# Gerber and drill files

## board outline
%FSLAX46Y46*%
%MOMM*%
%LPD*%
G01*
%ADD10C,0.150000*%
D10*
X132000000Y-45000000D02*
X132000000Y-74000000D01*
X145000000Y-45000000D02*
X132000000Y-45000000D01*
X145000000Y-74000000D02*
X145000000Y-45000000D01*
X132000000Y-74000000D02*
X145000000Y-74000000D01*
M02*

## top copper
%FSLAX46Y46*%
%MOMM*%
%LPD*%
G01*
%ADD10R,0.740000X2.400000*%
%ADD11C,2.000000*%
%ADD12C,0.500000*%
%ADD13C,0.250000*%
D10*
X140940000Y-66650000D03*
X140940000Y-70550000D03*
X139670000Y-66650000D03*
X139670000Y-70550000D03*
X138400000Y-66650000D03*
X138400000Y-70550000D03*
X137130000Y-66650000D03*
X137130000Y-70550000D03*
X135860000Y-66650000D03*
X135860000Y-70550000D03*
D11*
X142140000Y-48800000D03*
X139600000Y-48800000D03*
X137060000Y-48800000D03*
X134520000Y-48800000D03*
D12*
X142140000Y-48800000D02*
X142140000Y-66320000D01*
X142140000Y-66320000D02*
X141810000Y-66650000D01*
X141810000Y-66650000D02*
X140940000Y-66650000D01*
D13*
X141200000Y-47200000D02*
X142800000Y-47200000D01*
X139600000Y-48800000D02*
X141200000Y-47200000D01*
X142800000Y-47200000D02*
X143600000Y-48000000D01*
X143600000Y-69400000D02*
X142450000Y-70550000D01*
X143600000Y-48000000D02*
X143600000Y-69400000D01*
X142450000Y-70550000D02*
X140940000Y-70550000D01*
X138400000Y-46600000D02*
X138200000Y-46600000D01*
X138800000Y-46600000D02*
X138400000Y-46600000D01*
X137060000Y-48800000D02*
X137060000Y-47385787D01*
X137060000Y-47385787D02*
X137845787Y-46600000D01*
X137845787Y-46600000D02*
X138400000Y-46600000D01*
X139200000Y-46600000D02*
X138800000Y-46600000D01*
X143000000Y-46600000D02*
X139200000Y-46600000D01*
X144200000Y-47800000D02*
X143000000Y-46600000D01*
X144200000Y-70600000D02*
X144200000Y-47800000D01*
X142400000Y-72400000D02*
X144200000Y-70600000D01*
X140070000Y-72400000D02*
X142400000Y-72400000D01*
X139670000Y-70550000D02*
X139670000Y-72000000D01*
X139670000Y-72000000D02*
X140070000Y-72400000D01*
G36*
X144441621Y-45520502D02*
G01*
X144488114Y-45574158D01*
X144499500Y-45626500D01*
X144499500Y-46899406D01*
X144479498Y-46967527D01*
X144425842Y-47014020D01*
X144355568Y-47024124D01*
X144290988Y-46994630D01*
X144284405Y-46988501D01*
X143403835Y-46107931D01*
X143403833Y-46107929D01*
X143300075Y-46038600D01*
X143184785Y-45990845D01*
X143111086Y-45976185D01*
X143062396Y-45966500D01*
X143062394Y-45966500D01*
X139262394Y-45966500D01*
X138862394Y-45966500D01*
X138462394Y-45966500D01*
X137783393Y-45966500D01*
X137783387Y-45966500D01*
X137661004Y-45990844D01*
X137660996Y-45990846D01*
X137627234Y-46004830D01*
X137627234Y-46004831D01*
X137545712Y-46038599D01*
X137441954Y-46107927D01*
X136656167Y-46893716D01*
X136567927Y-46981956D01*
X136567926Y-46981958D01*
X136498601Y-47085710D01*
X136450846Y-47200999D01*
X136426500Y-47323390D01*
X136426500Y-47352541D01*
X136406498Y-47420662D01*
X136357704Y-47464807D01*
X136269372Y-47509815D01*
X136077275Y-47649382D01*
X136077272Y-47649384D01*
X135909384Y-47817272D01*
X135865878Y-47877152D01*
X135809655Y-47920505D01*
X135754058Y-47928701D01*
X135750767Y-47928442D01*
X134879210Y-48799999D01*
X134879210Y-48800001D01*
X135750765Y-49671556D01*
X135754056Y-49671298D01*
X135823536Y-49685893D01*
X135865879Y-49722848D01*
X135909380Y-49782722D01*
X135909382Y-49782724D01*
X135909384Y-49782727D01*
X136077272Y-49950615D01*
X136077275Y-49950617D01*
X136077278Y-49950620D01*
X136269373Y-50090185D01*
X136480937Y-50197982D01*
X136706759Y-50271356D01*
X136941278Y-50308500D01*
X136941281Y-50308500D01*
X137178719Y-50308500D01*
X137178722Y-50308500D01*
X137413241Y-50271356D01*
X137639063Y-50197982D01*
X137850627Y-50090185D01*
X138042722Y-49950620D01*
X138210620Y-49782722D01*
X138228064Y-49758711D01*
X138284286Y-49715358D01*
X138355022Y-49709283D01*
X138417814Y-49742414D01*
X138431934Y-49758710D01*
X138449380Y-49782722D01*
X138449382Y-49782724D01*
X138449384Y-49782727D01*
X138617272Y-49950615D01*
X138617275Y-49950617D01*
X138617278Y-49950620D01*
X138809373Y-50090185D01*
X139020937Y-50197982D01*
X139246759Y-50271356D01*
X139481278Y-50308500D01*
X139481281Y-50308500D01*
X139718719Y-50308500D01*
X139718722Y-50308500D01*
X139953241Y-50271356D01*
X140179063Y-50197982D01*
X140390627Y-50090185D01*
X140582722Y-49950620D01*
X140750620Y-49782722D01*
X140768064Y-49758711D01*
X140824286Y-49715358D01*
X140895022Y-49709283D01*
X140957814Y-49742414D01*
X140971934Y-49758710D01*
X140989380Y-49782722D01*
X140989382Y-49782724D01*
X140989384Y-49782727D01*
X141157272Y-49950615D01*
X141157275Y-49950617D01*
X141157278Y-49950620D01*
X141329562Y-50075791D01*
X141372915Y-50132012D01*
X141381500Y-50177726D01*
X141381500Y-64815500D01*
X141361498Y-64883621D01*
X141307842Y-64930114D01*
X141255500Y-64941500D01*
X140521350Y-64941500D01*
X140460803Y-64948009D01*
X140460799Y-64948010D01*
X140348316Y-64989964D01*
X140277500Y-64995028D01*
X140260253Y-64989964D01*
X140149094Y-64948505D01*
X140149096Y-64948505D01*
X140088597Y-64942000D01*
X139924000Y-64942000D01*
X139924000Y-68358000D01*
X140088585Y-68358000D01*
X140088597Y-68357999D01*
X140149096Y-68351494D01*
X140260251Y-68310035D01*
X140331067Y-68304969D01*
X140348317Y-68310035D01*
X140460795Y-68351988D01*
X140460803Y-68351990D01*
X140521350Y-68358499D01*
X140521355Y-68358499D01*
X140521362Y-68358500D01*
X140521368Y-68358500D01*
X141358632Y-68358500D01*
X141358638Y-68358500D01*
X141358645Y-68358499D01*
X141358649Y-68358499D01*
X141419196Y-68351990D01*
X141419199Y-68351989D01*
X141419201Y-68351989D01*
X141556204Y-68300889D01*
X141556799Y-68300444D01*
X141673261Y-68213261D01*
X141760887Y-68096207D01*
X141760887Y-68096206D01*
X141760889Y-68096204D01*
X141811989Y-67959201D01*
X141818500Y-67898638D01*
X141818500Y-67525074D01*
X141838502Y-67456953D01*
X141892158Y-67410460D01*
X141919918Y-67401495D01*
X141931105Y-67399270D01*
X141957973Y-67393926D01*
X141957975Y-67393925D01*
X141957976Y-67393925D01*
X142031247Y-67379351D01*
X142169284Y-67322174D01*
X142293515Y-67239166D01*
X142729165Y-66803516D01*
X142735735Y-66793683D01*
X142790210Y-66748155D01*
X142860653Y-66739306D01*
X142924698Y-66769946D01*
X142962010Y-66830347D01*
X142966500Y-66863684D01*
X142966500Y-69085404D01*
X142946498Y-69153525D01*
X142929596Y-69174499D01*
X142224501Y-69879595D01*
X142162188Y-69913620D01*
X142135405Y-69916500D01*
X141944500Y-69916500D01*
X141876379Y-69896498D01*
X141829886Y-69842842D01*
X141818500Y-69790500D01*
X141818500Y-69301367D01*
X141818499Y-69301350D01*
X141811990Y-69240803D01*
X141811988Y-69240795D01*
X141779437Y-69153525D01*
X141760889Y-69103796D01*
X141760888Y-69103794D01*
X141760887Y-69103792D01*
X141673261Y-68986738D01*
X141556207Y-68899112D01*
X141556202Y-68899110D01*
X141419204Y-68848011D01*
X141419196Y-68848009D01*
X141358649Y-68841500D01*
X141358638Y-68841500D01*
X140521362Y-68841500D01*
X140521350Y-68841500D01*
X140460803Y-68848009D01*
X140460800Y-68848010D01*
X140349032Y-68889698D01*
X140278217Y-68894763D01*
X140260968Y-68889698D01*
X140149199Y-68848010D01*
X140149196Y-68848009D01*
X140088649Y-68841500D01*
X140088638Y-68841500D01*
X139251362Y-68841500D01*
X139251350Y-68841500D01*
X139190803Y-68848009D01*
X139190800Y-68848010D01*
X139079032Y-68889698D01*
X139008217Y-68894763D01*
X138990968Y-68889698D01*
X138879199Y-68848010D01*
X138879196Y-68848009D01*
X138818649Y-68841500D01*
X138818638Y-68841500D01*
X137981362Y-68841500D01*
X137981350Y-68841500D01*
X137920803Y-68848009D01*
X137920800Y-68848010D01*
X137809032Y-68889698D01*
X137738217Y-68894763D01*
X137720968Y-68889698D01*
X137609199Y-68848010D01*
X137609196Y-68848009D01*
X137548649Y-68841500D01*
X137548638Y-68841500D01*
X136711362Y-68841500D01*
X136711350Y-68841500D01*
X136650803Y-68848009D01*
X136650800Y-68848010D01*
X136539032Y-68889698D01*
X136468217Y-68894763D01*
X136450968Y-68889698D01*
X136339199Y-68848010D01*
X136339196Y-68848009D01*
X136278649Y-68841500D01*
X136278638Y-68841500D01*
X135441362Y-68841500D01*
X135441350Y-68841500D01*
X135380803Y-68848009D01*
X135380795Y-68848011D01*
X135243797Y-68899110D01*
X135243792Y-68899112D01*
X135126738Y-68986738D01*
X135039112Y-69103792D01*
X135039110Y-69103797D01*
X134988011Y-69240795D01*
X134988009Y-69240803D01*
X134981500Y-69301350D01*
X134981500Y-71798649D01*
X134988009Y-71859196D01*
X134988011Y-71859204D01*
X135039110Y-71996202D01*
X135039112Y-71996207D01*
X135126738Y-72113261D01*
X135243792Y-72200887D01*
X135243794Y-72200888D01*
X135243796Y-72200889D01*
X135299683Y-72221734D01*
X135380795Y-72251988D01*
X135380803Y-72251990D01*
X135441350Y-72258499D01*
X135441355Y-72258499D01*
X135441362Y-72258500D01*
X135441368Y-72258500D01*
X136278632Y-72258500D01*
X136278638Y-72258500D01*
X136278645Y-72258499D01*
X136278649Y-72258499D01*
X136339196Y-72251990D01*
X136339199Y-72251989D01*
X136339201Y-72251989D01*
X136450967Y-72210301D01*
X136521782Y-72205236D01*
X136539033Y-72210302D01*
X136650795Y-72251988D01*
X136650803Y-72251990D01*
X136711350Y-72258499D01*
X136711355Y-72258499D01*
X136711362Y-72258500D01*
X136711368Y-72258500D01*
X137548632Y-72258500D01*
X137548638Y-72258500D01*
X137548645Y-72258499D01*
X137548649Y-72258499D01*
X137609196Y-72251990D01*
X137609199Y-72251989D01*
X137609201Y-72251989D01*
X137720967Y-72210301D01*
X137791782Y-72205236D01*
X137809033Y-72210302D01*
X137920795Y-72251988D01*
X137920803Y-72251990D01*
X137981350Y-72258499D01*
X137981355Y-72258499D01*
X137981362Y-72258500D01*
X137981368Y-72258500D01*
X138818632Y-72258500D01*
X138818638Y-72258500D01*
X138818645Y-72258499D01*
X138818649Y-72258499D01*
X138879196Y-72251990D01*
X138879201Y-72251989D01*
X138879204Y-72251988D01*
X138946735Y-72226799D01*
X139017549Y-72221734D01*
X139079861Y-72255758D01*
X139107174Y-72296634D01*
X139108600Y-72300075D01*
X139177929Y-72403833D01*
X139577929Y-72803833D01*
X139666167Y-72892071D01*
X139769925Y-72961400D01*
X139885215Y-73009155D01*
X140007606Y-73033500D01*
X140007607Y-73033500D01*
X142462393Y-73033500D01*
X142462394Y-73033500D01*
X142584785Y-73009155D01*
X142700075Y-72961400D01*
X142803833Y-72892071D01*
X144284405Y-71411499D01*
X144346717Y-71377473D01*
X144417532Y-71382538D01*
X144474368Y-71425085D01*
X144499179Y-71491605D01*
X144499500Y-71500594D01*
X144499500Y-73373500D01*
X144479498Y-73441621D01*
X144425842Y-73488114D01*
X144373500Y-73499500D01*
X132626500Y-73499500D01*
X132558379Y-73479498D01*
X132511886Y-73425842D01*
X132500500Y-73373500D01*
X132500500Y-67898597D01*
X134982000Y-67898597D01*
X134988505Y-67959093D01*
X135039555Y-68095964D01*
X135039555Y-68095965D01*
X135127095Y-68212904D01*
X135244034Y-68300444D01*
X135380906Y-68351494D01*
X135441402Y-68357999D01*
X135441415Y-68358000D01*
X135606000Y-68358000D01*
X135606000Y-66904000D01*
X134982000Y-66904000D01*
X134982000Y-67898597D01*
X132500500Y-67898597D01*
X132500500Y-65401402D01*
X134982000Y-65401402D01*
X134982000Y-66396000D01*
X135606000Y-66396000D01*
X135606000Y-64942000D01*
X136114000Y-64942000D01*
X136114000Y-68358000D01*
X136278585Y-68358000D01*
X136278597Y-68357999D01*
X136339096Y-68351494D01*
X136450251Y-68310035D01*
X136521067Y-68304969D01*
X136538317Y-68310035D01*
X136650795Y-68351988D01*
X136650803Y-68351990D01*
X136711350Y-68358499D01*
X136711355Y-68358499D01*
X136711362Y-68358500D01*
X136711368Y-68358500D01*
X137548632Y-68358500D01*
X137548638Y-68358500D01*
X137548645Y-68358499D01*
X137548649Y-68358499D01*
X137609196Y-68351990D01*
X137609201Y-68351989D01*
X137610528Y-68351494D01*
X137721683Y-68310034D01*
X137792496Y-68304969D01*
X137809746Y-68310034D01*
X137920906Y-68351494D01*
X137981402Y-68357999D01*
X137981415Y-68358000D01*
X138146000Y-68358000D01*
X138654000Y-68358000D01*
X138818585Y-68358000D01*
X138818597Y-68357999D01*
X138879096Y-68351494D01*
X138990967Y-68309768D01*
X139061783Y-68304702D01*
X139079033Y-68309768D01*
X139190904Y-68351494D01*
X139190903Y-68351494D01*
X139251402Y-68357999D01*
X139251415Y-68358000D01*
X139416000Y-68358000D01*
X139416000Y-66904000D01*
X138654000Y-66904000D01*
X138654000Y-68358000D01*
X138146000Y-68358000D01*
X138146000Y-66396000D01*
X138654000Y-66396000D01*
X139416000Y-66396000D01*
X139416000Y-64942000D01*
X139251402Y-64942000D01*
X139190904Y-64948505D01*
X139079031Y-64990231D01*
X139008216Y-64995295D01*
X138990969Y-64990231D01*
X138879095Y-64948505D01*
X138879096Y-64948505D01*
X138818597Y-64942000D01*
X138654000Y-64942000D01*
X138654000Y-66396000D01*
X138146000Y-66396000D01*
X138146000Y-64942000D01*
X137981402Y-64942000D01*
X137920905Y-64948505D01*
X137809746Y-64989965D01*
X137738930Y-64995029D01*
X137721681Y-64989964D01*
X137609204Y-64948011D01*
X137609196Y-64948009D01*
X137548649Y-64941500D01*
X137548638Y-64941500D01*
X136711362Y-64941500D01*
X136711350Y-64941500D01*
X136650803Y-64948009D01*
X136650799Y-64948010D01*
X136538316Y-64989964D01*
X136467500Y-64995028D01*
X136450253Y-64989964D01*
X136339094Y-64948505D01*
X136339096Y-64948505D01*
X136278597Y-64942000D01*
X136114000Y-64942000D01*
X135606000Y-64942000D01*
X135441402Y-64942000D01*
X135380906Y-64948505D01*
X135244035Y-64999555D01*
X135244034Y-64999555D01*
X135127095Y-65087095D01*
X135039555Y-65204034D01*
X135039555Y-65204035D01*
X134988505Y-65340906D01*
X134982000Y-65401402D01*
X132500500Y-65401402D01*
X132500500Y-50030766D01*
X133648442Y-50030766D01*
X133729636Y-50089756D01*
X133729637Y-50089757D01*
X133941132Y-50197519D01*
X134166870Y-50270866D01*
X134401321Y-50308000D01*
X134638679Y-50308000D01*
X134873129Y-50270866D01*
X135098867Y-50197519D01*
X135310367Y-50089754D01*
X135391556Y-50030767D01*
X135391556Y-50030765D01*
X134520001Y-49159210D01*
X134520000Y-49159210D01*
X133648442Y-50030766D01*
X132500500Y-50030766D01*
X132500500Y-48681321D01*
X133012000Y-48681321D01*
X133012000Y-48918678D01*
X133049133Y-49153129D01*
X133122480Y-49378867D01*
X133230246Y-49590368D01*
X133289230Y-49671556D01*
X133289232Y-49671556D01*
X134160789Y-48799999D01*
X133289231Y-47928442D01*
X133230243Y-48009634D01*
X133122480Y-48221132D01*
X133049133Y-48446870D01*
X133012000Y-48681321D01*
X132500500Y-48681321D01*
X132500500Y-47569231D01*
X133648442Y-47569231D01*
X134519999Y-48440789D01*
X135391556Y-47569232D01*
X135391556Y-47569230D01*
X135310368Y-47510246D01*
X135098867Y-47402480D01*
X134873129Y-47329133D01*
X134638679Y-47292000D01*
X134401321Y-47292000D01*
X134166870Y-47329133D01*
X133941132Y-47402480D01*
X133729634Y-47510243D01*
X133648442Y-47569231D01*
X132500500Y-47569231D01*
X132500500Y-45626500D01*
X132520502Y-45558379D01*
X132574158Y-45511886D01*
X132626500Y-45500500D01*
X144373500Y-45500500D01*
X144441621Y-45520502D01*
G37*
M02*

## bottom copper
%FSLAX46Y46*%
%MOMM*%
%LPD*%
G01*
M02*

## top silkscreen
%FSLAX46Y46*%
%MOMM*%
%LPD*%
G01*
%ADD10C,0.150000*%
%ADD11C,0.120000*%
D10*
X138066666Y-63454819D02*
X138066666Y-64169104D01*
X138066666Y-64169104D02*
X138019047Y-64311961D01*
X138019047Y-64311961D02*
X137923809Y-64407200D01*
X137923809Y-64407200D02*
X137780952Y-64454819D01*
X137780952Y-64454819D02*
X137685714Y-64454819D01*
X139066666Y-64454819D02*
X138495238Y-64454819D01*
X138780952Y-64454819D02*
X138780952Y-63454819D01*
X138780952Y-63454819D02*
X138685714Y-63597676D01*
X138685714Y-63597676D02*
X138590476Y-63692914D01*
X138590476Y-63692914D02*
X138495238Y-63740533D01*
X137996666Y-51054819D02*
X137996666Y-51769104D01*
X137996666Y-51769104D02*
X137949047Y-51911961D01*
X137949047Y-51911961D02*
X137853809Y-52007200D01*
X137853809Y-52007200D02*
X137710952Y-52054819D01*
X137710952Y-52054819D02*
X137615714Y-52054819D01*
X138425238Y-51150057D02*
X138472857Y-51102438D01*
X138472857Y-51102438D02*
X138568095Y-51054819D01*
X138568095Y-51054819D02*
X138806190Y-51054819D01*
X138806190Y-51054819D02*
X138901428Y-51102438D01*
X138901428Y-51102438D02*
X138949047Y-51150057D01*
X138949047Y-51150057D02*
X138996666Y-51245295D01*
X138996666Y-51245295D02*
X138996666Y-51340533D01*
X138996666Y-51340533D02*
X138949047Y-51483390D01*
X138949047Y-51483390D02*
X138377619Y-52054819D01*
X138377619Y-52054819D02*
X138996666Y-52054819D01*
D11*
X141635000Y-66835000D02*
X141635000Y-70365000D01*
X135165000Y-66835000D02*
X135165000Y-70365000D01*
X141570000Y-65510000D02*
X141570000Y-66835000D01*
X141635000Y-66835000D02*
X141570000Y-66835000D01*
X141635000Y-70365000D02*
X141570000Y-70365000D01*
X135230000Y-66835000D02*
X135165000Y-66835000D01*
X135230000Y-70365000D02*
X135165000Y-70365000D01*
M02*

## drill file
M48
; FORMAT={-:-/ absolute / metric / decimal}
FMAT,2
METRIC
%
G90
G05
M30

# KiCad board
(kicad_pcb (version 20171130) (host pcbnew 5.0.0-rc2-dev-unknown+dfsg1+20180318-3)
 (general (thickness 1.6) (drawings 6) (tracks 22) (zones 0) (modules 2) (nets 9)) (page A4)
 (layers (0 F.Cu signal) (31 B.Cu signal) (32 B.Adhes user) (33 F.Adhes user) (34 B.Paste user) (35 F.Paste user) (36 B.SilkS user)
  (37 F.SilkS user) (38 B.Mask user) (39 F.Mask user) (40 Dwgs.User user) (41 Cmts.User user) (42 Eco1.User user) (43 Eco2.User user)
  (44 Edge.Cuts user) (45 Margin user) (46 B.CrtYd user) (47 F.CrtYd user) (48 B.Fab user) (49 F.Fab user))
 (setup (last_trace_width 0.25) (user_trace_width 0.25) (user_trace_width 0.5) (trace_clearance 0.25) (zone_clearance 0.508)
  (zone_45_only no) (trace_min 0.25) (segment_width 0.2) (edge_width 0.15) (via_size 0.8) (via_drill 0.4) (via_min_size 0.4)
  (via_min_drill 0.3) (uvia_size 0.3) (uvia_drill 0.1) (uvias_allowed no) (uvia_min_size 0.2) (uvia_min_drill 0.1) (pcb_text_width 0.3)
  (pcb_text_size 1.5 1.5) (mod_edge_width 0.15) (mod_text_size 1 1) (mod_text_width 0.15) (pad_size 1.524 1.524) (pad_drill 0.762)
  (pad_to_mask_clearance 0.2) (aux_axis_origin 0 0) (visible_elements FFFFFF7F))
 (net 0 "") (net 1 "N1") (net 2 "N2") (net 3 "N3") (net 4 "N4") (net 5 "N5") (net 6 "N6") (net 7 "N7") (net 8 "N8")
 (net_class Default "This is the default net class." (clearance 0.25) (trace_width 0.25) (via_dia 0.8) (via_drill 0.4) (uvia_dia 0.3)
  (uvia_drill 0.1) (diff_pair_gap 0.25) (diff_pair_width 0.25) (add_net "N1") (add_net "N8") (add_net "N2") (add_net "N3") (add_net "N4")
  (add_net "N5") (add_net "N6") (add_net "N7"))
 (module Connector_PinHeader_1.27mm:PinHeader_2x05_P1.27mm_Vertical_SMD (layer F.Cu) (at 138.4 68.6 270)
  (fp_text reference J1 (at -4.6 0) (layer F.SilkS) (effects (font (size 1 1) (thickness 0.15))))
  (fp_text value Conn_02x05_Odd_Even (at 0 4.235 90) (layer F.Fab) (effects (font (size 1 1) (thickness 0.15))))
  (fp_line (start -1.765 -3.235) (end 1.765 -3.235) (layer F.SilkS) (width 0.12))
  (fp_line (start -1.765 3.235) (end 1.765 3.235) (layer F.SilkS) (width 0.12))
  (fp_line (start -3.09 -3.17) (end -1.765 -3.17) (layer F.SilkS) (width 0.12))
  (fp_line (start -1.765 -3.235) (end -1.765 -3.17) (layer F.SilkS) (width 0.12))
  (fp_line (start 1.765 -3.235) (end 1.765 -3.17) (layer F.SilkS) (width 0.12))
  (fp_line (start -1.765 3.17) (end -1.765 3.235) (layer F.SilkS) (width 0.12))
  (fp_line (start 1.765 3.17) (end 1.765 3.235) (layer F.SilkS) (width 0.12))
  (pad 1 smd rect (at -1.95 -2.54 270) (size 2.4 0.74) (layers F.Cu F.Paste F.Mask) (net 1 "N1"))
  (pad 2 smd rect (at 1.95 -2.54 270) (size 2.4 0.74) (layers F.Cu F.Paste F.Mask) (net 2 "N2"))
  (pad 3 smd rect (at -1.95 -1.27 270) (size 2.4 0.74) (layers F.Cu F.Paste F.Mask) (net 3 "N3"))
  (pad 4 smd rect (at 1.95 -1.27 270) (size 2.4 0.74) (layers F.Cu F.Paste F.Mask) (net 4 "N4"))
  (pad 5 smd rect (at -1.95 0 270) (size 2.4 0.74) (layers F.Cu F.Paste F.Mask) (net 3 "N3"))
  (pad 6 smd rect (at 1.95 0 270) (size 2.4 0.74) (layers F.Cu F.Paste F.Mask) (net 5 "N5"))
  (pad 7 smd rect (at -1.95 1.27 270) (size 2.4 0.74) (layers F.Cu F.Paste F.Mask) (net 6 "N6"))
  (pad 8 smd rect (at 1.95 1.27 270) (size 2.4 0.74) (layers F.Cu F.Paste F.Mask) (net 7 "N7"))
  (pad 9 smd rect (at -1.95 2.54 270) (size 2.4 0.74) (layers F.Cu F.Paste F.Mask) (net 3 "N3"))
  (pad 10 smd rect (at 1.95 2.54 270) (size 2.4 0.74) (layers F.Cu F.Paste F.Mask) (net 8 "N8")))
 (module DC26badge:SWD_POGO (layer F.Cu) (at 138.33 48.8 180)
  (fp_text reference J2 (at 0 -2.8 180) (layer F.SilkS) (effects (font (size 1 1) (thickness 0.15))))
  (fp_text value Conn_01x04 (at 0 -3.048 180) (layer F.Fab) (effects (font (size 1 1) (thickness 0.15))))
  (pad 1 smd circle (at -3.81 0 180) (size 2 2) (layers F.Cu F.Paste F.Mask) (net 1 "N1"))
  (pad 2 smd circle (at -1.27 0 180) (size 2 2) (layers F.Cu F.Paste F.Mask) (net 2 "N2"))
  (pad 3 smd circle (at 1.27 0 180) (size 2 2) (layers F.Cu F.Paste F.Mask) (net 4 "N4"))
  (pad 4 smd circle (at 3.81 0 180) (size 2 2) (layers F.Cu F.Paste F.Mask) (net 3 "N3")))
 (gr_line (start 132 45) (end 132 74) (layer Edge.Cuts) (width 0.15))
 (gr_line (start 145 45) (end 132 45) (layer Edge.Cuts) (width 0.15))
 (gr_line (start 145 74) (end 145 45) (layer Edge.Cuts) (width 0.15))
 (gr_line (start 132 74) (end 145 74) (layer Edge.Cuts) (width 0.15))
 (segment (start 142.14 48.8) (end 142.14 66.32) (width 0.5) (layer F.Cu) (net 1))
 (segment (start 142.14 66.32) (end 141.81 66.65) (width 0.5) (layer F.Cu) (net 1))
 (segment (start 141.81 66.65) (end 140.94 66.65) (width 0.5) (layer F.Cu) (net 1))
 (segment (start 141.2 47.2) (end 142.8 47.2) (width 0.25) (layer F.Cu) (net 2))
 (segment (start 139.6 48.8) (end 141.2 47.2) (width 0.25) (layer F.Cu) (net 2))
 (segment (start 142.8 47.2) (end 143.6 48) (width 0.25) (layer F.Cu) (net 2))
 (segment (start 143.6 69.4) (end 142.45 70.55) (width 0.25) (layer F.Cu) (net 2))
 (segment (start 143.6 48) (end 143.6 69.4) (width 0.25) (layer F.Cu) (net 2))
 (segment (start 142.45 70.55) (end 140.94 70.55) (width 0.25) (layer F.Cu) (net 2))
 (segment (start 138.4 46.6) (end 138.2 46.6) (width 0.25) (layer F.Cu) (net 4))
 (segment (start 138.8 46.6) (end 138.4 46.6) (width 0.25) (layer F.Cu) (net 4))
 (segment (start 137.06 48.8) (end 137.06 47.385787) (width 0.25) (layer F.Cu) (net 4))
 (segment (start 137.06 47.385787) (end 137.845787 46.6) (width 0.25) (layer F.Cu) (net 4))
 (segment (start 137.845787 46.6) (end 138.4 46.6) (width 0.25) (layer F.Cu) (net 4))
 (segment (start 139.2 46.6) (end 138.8 46.6) (width 0.25) (layer F.Cu) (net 4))
 (segment (start 143 46.6) (end 139.2 46.6) (width 0.25) (layer F.Cu) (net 4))
 (segment (start 144.2 47.8) (end 143 46.6) (width 0.25) (layer F.Cu) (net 4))
 (segment (start 144.2 70.6) (end 144.2 47.8) (width 0.25) (layer F.Cu) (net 4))
 (segment (start 142.4 72.4) (end 144.2 70.6) (width 0.25) (layer F.Cu) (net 4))
 (segment (start 140.07 72.4) (end 142.4 72.4) (width 0.25) (layer F.Cu) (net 4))
 (segment (start 139.67 70.55) (end 139.67 72) (width 0.25) (layer F.Cu) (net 4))
 (segment (start 139.67 72) (end 140.07 72.4) (width 0.25) (layer F.Cu) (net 4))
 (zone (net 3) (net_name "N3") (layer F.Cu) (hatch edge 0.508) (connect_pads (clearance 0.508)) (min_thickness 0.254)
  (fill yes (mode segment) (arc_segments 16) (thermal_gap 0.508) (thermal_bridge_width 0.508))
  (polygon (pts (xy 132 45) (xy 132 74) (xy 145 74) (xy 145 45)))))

